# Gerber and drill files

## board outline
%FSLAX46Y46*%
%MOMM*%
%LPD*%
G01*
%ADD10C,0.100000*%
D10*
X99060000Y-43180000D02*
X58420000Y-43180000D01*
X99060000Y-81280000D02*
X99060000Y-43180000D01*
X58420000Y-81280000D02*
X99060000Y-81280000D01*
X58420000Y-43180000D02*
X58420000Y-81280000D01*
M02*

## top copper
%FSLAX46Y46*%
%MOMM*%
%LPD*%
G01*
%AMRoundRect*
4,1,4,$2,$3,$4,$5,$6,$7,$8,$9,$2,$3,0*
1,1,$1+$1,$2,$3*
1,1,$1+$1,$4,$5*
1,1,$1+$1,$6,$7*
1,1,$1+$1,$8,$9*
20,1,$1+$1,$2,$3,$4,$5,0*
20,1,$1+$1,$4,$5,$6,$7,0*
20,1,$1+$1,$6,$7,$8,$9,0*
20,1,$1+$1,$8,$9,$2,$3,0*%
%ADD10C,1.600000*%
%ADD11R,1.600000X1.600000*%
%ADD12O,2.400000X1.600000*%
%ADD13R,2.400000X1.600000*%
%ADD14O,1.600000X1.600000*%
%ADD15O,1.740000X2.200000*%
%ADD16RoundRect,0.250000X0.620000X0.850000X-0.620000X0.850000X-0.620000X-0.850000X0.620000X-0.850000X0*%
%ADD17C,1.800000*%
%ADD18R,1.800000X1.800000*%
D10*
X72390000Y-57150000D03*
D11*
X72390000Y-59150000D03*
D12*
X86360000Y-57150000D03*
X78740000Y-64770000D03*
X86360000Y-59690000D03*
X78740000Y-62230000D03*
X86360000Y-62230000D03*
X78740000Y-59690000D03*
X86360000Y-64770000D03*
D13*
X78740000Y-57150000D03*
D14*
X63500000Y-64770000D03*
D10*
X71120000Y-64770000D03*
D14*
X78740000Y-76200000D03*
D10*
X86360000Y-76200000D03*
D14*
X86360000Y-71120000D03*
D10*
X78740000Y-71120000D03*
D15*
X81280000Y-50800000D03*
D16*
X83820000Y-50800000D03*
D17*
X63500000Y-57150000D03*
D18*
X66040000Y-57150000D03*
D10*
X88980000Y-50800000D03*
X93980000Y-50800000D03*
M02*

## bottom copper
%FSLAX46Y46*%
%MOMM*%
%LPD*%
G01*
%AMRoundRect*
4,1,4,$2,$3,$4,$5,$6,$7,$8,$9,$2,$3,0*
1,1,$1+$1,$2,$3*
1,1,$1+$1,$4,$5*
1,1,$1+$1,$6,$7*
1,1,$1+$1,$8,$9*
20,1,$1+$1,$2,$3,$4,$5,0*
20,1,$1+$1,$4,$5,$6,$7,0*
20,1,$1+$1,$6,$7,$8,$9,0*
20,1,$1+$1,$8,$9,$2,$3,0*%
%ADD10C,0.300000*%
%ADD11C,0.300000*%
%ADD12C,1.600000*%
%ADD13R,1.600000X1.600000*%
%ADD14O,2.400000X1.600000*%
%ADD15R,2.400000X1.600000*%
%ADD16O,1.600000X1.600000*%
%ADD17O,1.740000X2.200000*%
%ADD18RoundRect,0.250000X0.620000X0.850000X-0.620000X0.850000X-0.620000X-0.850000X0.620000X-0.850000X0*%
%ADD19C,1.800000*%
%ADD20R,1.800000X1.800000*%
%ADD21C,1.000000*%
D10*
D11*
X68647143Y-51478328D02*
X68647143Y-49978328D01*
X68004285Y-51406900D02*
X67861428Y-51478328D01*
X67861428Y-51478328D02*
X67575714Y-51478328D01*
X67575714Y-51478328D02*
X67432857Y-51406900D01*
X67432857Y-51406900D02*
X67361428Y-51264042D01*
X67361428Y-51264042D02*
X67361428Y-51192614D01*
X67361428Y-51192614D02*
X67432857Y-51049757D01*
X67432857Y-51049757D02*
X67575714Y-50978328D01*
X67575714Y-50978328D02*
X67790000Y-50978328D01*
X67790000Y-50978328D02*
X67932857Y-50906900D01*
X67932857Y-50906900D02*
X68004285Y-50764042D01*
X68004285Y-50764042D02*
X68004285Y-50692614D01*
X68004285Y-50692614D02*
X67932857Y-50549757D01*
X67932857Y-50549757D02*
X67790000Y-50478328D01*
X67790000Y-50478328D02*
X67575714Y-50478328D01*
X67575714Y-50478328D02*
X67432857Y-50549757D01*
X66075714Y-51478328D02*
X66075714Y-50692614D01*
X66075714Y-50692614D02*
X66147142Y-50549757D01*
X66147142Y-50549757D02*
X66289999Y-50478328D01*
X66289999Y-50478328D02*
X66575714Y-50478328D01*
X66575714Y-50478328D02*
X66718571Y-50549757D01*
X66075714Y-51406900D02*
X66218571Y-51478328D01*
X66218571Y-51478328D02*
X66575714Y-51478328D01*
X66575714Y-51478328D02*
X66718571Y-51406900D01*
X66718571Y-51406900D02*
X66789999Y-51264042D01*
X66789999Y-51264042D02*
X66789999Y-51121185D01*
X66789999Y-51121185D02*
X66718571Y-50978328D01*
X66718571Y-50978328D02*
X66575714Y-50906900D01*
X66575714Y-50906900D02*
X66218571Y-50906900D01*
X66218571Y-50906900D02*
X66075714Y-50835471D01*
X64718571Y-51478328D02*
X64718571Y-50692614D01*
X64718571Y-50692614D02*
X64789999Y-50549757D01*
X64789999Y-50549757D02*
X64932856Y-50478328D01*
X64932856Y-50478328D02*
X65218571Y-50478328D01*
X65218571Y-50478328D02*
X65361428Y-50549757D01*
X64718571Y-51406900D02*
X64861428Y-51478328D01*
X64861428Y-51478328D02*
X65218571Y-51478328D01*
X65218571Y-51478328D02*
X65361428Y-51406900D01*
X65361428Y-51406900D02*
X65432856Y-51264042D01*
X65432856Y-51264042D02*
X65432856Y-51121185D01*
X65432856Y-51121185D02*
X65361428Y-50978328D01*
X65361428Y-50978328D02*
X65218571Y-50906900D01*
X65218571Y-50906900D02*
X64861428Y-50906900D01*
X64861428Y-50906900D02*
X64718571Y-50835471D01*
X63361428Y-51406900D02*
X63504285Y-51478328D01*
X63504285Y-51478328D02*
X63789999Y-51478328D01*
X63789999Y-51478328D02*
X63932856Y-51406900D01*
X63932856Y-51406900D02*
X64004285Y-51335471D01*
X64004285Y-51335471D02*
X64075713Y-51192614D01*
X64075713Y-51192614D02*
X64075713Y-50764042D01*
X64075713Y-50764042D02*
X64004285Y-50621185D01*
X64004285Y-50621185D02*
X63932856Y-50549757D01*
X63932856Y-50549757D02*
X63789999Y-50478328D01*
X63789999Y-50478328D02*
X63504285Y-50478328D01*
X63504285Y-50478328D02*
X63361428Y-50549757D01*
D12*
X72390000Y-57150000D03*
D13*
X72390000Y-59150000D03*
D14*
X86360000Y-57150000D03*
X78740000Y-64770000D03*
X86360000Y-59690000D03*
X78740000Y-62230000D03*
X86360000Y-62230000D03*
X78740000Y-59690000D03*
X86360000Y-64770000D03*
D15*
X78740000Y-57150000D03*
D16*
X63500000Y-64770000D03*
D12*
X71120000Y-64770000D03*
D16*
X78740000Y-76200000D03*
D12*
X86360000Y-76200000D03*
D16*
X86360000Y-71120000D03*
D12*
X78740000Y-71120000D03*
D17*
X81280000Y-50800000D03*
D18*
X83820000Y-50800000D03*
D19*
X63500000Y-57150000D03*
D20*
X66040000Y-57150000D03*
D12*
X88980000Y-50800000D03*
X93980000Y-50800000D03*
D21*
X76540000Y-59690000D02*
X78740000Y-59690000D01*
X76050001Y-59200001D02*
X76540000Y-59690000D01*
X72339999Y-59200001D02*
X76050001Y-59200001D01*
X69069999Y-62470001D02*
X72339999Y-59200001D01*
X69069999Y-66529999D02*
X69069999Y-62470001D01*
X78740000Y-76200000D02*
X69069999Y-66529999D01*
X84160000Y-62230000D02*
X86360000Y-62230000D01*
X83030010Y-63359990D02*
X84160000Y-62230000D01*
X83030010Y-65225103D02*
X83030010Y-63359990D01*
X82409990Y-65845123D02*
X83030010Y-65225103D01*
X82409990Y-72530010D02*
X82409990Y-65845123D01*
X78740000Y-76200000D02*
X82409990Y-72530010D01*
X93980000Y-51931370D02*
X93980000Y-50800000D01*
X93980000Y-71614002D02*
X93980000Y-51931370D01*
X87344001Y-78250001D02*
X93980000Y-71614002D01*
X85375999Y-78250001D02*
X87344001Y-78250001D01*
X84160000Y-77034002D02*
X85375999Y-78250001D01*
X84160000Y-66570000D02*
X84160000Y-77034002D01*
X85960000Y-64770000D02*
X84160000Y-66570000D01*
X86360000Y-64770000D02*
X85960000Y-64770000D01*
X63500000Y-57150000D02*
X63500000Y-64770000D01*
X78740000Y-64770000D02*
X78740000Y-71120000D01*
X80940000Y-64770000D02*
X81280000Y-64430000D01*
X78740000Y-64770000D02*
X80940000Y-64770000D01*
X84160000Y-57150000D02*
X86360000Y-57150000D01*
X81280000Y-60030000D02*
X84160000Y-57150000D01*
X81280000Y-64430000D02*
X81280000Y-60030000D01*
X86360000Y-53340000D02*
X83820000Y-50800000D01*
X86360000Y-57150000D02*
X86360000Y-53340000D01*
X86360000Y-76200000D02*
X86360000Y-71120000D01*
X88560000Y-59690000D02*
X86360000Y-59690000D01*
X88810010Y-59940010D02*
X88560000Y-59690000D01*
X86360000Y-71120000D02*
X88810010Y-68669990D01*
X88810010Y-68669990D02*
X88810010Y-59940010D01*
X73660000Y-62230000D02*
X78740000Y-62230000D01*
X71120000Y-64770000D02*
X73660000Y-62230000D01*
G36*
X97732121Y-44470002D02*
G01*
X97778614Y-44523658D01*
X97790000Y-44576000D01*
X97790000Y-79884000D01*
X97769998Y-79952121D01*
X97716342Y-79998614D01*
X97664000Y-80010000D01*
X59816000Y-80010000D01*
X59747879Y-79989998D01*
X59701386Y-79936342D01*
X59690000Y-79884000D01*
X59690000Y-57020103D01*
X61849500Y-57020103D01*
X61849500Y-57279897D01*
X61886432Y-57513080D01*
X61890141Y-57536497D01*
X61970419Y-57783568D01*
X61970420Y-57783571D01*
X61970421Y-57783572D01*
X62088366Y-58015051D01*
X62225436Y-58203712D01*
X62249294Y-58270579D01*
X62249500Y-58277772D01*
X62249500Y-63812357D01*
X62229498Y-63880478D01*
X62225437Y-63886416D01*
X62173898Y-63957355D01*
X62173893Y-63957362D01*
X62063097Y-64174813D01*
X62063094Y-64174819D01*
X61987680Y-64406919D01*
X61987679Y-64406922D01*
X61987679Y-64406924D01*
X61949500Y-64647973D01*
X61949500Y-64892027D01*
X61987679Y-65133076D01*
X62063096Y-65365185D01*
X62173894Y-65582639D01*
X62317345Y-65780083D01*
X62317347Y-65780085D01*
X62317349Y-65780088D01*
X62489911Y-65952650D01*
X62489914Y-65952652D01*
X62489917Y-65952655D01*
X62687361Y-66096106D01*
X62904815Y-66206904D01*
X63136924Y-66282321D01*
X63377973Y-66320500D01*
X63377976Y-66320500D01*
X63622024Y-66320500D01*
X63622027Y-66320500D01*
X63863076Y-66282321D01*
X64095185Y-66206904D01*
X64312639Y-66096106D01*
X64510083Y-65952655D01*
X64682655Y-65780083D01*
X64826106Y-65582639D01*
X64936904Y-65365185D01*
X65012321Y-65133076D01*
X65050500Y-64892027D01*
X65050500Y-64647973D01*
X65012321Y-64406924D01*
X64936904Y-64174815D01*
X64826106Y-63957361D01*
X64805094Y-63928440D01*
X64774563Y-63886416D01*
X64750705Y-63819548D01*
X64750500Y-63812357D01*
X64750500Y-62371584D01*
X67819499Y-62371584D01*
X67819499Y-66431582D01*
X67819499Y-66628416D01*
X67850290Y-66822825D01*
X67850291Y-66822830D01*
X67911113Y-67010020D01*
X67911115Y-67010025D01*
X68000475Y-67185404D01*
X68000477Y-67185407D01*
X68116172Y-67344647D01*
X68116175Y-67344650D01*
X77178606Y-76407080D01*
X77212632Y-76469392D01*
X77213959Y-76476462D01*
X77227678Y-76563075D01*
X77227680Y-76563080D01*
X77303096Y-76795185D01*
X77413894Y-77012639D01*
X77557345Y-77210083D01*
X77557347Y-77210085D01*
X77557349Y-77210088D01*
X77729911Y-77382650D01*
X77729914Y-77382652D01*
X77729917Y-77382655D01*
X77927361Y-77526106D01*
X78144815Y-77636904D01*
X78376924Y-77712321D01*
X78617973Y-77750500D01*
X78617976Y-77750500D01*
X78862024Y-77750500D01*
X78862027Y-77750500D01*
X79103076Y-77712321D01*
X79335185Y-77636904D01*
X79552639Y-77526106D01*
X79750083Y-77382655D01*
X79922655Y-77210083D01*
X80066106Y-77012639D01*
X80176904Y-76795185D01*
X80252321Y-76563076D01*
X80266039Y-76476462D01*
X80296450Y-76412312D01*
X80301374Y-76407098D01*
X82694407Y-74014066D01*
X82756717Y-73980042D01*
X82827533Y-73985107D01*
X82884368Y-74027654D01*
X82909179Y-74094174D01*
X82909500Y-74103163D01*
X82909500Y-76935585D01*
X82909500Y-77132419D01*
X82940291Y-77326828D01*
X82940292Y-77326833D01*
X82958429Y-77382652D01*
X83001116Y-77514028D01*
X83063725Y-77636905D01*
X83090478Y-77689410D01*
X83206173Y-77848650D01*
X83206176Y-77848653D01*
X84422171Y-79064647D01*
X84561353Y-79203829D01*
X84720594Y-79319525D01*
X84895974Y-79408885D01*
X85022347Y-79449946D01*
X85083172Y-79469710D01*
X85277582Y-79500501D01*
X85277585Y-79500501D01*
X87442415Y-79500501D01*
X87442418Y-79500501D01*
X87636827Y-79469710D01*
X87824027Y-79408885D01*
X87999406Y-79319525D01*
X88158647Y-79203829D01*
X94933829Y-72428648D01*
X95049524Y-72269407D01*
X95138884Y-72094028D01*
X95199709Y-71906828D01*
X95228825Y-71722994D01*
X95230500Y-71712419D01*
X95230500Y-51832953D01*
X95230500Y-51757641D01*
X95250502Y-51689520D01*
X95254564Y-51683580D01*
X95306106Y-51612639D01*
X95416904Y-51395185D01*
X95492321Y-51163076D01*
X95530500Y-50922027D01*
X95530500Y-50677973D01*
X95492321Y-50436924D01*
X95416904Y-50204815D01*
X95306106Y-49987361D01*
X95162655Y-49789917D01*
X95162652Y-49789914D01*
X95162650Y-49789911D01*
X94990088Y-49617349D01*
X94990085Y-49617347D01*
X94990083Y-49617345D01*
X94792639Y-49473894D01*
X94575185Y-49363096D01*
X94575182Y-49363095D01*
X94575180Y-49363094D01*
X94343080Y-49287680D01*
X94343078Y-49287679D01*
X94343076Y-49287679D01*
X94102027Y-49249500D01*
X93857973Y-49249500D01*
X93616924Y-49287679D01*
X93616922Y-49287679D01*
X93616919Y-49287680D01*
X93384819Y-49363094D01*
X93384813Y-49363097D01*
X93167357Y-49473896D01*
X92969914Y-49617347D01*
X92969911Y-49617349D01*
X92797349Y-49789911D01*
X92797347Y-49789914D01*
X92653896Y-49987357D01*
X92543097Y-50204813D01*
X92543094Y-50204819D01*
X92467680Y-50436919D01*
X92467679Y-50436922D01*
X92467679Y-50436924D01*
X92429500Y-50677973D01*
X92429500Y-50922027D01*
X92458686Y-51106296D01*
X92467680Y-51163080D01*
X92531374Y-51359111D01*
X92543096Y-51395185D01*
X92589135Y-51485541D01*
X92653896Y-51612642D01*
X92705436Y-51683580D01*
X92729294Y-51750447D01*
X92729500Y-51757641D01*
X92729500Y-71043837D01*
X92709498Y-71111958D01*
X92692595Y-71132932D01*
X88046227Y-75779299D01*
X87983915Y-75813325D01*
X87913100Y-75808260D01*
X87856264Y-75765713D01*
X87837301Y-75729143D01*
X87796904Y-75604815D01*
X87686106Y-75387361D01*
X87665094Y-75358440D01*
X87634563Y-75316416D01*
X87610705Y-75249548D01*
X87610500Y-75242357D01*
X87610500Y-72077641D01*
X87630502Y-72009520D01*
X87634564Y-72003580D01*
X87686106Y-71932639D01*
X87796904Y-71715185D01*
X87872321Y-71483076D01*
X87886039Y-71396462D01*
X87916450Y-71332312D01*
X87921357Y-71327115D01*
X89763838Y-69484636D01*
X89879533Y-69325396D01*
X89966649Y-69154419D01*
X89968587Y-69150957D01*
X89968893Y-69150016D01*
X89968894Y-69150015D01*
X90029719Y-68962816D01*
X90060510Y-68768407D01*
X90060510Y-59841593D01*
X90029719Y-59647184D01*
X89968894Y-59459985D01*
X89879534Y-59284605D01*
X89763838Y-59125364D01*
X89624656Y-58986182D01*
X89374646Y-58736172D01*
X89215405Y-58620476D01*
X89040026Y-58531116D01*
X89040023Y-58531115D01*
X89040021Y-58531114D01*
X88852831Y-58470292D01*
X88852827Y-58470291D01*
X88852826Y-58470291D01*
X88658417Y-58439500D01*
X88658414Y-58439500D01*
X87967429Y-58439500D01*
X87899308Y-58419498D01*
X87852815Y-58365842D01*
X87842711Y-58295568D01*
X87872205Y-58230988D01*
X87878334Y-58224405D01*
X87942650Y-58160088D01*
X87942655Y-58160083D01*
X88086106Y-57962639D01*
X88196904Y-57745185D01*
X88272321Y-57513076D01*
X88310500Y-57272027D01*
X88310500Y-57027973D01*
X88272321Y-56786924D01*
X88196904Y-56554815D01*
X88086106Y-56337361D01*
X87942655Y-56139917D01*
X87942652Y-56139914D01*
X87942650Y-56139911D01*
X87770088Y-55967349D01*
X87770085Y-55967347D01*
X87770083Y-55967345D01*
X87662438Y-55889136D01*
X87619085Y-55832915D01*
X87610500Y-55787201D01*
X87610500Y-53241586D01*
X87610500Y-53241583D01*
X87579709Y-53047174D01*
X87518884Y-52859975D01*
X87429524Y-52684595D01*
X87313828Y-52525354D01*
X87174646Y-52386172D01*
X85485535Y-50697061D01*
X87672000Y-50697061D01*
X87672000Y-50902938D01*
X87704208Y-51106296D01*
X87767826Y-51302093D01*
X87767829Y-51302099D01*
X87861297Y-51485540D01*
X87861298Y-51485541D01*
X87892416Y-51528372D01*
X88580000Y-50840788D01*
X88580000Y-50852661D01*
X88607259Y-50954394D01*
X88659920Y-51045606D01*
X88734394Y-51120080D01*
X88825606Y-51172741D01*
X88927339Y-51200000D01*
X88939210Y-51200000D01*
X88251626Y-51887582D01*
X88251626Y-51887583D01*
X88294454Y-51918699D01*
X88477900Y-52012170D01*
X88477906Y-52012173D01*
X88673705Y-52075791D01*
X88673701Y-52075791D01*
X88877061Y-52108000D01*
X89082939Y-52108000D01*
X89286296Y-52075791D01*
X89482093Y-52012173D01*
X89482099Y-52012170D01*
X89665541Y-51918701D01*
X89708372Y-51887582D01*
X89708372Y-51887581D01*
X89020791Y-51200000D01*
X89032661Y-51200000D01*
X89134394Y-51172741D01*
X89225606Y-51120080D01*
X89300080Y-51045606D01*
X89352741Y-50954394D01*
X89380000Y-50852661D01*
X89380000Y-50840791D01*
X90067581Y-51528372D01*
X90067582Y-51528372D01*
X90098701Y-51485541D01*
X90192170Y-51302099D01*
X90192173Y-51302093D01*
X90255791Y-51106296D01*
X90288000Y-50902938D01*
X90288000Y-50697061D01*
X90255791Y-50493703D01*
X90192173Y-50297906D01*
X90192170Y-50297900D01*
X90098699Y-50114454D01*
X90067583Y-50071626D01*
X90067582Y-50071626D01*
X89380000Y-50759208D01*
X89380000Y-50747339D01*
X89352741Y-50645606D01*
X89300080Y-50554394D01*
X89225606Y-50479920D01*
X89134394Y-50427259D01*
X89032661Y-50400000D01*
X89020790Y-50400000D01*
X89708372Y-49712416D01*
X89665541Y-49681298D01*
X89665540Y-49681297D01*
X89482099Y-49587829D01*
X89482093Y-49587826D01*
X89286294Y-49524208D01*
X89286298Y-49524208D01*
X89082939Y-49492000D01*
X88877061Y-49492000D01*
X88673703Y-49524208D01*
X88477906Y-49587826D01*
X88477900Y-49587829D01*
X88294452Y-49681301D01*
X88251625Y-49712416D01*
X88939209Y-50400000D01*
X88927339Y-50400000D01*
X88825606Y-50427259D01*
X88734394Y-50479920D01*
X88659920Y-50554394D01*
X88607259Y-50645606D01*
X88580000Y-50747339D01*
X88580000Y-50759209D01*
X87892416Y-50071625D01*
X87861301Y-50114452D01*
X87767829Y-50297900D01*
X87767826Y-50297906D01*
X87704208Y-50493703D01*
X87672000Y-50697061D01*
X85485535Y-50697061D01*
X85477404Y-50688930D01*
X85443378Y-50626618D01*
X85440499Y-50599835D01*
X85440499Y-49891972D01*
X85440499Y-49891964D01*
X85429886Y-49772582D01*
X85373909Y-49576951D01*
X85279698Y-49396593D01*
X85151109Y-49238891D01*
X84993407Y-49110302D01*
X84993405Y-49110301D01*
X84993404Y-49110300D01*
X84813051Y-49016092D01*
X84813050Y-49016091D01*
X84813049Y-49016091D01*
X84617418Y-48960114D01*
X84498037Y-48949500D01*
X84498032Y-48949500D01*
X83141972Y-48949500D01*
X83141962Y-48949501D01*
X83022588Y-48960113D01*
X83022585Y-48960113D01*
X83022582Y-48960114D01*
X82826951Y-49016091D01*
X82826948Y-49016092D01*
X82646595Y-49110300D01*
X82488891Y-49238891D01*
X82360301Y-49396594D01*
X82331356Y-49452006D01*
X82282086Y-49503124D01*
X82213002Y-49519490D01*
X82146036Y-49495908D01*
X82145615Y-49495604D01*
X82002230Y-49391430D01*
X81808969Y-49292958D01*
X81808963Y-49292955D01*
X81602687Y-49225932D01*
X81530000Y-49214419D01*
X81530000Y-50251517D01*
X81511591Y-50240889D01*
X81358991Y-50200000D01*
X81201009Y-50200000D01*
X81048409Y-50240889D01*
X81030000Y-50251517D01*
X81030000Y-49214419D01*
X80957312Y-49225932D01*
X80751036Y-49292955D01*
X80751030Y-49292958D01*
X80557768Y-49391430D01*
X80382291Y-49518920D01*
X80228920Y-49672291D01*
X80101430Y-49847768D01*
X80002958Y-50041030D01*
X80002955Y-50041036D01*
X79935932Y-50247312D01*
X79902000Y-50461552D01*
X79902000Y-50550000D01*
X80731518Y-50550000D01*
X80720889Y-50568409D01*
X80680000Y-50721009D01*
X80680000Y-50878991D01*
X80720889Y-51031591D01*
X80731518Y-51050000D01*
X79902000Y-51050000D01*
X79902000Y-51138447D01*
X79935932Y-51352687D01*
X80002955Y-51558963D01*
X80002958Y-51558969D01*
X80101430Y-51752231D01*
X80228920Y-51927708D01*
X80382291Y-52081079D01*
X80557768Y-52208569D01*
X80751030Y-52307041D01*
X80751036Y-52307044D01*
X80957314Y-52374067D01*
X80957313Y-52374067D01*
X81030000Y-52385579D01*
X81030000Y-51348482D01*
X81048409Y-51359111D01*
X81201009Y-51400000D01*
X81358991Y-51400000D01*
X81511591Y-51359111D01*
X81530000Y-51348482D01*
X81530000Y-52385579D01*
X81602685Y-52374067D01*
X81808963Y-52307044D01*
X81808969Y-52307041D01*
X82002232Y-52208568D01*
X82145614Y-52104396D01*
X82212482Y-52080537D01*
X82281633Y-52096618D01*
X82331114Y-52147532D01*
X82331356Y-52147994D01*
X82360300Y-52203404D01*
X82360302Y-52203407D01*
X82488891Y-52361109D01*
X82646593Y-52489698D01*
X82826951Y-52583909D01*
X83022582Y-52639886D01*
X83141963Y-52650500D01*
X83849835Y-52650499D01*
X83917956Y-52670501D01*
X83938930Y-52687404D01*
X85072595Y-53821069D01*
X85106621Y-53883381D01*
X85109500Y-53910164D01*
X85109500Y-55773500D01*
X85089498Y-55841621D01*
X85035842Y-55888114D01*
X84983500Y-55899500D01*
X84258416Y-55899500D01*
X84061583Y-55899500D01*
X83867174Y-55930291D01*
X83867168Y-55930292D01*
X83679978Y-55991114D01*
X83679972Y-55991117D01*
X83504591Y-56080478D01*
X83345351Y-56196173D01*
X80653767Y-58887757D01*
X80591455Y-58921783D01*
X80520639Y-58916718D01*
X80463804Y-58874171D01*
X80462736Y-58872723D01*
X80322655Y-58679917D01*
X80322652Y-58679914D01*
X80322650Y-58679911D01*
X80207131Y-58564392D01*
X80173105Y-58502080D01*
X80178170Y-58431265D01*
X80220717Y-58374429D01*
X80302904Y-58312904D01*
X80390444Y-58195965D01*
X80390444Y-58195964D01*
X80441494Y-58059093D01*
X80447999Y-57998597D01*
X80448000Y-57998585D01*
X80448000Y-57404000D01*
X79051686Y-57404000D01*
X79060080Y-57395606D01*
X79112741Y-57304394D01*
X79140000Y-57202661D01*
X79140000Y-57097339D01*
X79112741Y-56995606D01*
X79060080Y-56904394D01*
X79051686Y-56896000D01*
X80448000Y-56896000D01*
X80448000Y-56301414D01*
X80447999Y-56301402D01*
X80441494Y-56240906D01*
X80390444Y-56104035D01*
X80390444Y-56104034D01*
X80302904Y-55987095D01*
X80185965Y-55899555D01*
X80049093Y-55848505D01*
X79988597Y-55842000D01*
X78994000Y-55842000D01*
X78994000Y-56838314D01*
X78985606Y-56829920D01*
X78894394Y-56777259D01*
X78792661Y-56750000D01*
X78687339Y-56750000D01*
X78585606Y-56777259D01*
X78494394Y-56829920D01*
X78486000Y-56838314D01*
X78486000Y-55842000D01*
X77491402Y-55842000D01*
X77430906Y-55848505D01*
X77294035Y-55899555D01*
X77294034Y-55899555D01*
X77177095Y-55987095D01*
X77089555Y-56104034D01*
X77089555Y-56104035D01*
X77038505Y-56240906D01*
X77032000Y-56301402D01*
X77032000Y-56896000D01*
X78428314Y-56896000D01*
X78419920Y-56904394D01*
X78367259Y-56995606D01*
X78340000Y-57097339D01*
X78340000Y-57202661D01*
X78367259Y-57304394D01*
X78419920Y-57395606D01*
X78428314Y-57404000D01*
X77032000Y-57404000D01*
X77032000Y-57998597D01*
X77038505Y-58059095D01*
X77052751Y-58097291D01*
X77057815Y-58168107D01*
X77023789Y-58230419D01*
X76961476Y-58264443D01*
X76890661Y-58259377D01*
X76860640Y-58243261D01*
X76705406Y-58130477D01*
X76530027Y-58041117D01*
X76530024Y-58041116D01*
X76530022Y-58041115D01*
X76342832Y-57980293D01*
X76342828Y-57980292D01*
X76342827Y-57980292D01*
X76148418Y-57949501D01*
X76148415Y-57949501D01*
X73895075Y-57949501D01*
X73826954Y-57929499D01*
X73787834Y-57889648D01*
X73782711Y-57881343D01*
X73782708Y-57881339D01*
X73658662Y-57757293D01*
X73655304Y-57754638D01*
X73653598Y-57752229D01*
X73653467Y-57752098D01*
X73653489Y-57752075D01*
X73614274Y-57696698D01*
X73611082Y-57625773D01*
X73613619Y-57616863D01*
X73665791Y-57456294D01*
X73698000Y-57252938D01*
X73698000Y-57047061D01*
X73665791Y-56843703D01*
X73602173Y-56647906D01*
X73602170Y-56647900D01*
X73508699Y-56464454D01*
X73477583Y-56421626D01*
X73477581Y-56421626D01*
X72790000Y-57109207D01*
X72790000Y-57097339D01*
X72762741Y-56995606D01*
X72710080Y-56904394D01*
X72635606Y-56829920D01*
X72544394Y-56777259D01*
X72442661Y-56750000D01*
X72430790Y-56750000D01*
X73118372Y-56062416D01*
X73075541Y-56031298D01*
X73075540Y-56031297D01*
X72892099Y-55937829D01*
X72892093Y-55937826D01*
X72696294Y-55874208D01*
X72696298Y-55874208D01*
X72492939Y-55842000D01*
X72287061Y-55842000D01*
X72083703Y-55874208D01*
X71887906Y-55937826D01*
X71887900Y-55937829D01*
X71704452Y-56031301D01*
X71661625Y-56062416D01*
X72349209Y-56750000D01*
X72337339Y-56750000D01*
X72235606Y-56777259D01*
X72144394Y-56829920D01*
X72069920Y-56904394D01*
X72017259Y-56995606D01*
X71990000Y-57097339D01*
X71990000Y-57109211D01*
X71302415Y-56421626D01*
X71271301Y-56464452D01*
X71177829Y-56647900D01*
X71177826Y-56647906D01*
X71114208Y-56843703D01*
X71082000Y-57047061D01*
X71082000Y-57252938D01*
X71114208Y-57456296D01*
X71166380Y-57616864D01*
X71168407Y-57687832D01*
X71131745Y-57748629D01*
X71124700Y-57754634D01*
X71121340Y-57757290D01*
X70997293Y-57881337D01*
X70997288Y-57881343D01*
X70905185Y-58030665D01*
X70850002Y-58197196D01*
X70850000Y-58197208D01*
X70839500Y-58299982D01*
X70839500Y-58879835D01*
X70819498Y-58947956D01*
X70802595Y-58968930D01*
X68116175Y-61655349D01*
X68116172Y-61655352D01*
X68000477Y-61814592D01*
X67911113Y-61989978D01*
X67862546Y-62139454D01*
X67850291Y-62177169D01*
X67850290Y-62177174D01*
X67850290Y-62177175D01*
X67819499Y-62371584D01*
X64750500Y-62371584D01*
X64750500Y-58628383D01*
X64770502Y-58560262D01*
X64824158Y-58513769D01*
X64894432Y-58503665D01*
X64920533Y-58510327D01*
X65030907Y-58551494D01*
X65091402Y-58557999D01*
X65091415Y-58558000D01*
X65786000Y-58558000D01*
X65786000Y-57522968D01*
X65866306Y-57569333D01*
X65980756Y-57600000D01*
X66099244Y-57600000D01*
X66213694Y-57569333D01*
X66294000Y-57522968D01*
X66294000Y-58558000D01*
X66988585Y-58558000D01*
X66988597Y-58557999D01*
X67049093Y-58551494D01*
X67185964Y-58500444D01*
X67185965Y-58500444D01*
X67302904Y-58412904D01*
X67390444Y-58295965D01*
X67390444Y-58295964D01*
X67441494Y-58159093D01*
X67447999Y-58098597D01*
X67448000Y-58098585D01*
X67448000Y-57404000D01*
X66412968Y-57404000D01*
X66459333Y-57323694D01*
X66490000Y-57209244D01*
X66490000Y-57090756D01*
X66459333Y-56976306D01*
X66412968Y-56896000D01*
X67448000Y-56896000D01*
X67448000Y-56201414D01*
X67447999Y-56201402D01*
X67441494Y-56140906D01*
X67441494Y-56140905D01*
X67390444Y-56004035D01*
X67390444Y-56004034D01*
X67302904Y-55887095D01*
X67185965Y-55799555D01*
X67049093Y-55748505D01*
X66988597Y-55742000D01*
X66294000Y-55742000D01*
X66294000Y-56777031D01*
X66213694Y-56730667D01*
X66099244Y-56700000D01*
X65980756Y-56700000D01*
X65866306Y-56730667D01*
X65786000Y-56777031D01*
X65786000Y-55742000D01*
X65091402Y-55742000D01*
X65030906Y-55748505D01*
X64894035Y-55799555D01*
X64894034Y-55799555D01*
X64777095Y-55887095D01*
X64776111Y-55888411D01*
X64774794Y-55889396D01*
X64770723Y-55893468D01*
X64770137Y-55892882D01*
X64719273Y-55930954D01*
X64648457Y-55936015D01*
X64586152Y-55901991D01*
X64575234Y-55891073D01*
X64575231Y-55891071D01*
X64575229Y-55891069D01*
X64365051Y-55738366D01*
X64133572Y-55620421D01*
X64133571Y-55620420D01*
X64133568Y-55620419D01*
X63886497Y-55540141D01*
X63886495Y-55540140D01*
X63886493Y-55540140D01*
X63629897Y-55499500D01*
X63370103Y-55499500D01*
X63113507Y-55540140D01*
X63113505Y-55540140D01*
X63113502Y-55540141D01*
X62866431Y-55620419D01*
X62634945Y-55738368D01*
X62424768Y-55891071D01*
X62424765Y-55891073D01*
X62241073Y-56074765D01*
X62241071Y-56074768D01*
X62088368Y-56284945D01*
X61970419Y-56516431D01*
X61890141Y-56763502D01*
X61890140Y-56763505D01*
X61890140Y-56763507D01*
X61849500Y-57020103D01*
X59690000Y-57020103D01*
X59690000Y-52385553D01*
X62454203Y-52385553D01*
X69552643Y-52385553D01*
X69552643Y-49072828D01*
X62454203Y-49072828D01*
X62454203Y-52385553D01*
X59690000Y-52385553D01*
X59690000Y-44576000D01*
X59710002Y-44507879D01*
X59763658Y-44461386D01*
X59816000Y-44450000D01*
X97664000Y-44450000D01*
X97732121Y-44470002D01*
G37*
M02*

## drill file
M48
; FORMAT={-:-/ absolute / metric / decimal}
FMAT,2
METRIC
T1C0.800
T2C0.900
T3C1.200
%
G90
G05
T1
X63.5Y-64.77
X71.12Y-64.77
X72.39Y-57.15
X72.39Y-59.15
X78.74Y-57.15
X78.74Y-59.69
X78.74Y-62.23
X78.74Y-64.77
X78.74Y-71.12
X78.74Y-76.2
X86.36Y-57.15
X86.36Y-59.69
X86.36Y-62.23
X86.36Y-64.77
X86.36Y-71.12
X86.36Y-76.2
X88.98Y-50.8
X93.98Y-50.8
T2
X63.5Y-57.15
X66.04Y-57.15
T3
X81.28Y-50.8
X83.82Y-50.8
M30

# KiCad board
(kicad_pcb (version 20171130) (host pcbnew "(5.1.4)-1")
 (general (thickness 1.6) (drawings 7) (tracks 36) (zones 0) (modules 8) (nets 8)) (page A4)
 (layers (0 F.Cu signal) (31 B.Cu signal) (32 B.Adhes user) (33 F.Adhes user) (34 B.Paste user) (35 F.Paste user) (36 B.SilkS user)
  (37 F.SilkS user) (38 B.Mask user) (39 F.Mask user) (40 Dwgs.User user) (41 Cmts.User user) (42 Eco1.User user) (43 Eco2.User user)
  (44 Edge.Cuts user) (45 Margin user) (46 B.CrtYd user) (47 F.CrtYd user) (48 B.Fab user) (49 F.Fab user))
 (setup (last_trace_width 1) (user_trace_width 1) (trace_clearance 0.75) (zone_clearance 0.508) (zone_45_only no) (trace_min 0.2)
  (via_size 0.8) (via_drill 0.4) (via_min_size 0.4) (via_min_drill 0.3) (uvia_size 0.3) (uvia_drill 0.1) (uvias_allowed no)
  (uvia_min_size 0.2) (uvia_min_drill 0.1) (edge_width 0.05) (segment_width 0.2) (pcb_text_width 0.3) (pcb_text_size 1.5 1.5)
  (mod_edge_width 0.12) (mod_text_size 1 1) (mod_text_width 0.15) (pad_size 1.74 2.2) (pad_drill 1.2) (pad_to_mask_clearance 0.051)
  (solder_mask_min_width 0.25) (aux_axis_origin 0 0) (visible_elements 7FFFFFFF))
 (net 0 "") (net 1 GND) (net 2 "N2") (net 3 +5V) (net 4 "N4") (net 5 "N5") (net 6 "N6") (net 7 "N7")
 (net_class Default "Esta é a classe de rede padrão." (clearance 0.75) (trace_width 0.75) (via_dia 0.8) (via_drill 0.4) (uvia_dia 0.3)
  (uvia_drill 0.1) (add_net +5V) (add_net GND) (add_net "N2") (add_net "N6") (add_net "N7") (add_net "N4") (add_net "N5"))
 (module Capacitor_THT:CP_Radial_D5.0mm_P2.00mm (layer F.Cu) (at 72.39 59.15 90)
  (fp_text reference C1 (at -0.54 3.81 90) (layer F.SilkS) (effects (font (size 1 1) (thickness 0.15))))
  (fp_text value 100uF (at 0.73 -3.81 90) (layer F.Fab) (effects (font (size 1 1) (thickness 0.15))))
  (pad 2 thru_hole circle (at 2 0 90) (size 1.6 1.6) (drill 0.8) (layers *.Cu *.Mask) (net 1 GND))
  (pad 1 thru_hole rect (at 0 0 90) (size 1.6 1.6) (drill 0.8) (layers *.Cu *.Mask) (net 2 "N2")))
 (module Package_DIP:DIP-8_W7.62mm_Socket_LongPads (layer F.Cu) (at 78.74 57.15)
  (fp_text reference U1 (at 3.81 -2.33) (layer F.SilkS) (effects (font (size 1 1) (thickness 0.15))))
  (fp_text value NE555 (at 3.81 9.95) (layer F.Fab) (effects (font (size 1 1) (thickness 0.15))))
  (pad 8 thru_hole oval (at 7.62 0) (size 2.4 1.6) (drill 0.8) (layers *.Cu *.Mask) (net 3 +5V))
  (pad 4 thru_hole oval (at 0 7.62) (size 2.4 1.6) (drill 0.8) (layers *.Cu *.Mask) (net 3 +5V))
  (pad 7 thru_hole oval (at 7.62 2.54) (size 2.4 1.6) (drill 0.8) (layers *.Cu *.Mask) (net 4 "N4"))
  (pad 3 thru_hole oval (at 0 5.08) (size 2.4 1.6) (drill 0.8) (layers *.Cu *.Mask) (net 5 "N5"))
  (pad 6 thru_hole oval (at 7.62 5.08) (size 2.4 1.6) (drill 0.8) (layers *.Cu *.Mask) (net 2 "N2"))
  (pad 2 thru_hole oval (at 0 2.54) (size 2.4 1.6) (drill 0.8) (layers *.Cu *.Mask) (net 2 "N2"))
  (pad 5 thru_hole oval (at 7.62 7.62) (size 2.4 1.6) (drill 0.8) (layers *.Cu *.Mask) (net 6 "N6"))
  (pad 1 thru_hole rect (at 0 0) (size 2.4 1.6) (drill 0.8) (layers *.Cu *.Mask) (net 1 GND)))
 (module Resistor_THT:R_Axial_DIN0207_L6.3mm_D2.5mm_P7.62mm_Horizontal (layer F.Cu) (at 71.12 64.77 180)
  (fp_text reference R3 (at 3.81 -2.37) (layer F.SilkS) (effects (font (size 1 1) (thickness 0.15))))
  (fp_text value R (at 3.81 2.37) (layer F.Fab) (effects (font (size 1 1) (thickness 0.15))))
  (pad 2 thru_hole oval (at 7.62 0 180) (size 1.6 1.6) (drill 0.8) (layers *.Cu *.Mask) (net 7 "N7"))
  (pad 1 thru_hole circle (at 0 0 180) (size 1.6 1.6) (drill 0.8) (layers *.Cu *.Mask) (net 5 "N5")))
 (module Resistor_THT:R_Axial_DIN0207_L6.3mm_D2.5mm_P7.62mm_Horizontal (layer F.Cu) (at 86.36 76.2 180)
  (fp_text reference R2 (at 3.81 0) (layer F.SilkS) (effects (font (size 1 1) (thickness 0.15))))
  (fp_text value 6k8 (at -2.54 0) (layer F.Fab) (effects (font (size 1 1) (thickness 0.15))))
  (pad 2 thru_hole oval (at 7.62 0 180) (size 1.6 1.6) (drill 0.8) (layers *.Cu *.Mask) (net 2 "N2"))
  (pad 1 thru_hole circle (at 0 0 180) (size 1.6 1.6) (drill 0.8) (layers *.Cu *.Mask) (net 4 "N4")))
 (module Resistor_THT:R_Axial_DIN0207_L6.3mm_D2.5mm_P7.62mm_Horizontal (layer F.Cu) (at 78.74 71.12)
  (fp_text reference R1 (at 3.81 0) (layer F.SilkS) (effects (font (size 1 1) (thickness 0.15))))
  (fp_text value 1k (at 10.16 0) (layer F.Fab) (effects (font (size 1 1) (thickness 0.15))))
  (pad 2 thru_hole oval (at 7.62 0) (size 1.6 1.6) (drill 0.8) (layers *.Cu *.Mask) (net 4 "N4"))
  (pad 1 thru_hole circle (at 0 0) (size 1.6 1.6) (drill 0.8) (layers *.Cu *.Mask) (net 3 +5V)))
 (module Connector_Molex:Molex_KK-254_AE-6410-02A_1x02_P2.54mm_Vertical (layer F.Cu) (at 83.82 50.8 180)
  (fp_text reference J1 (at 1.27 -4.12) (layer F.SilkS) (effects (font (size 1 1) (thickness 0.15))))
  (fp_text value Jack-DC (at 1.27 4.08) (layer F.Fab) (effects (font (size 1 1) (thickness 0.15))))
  (pad 2 thru_hole oval (at 2.54 0 180) (size 1.74 2.2) (drill 1.2) (layers *.Cu *.Mask) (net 1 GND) (thermal_width 0.5))
  (pad 1 thru_hole roundrect (at 0 0 180) (size 1.74 2.2) (drill 1.2) (layers *.Cu *.Mask) (roundrect_rratio 0.143678) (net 3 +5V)))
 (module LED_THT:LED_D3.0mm (layer F.Cu) (at 66.04 57.15 180)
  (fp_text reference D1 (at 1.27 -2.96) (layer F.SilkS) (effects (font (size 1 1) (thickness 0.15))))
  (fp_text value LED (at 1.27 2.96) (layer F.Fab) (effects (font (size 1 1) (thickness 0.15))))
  (pad 2 thru_hole circle (at 2.54 0 180) (size 1.8 1.8) (drill 0.9) (layers *.Cu *.Mask) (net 7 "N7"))
  (pad 1 thru_hole rect (at 0 0 180) (size 1.8 1.8) (drill 0.9) (layers *.Cu *.Mask) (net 1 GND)))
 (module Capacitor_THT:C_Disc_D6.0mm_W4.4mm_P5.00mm (layer F.Cu) (at 93.98 50.8 180)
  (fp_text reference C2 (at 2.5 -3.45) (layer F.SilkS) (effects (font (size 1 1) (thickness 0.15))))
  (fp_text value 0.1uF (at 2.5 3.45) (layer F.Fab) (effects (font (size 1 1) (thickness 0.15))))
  (pad 2 thru_hole circle (at 5 0 180) (size 1.6 1.6) (drill 0.8) (layers *.Cu *.Mask) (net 1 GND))
  (pad 1 thru_hole circle (at 0 0 180) (size 1.6 1.6) (drill 0.8) (layers *.Cu *.Mask) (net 6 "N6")))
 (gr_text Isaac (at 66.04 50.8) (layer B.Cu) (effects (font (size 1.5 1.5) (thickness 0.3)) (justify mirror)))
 (gr_line (start 99.06 43.18) (end 58.42 43.18) (layer Edge.Cuts) (width 0.1))
 (gr_line (start 99.06 81.28) (end 99.06 43.18) (layer Edge.Cuts) (width 0.1))
 (gr_line (start 58.42 81.28) (end 99.06 81.28) (layer Edge.Cuts) (width 0.1))
 (gr_line (start 58.42 43.18) (end 58.42 81.28) (layer Edge.Cuts) (width 0.1))
 (segment (start 76.54 59.69) (end 78.74 59.69) (width 1) (layer B.Cu) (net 2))
 (segment (start 76.050001 59.200001) (end 76.54 59.69) (width 1) (layer B.Cu) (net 2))
 (segment (start 72.339999 59.200001) (end 76.050001 59.200001) (width 1) (layer B.Cu) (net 2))
 (segment (start 69.069999 62.470001) (end 72.339999 59.200001) (width 1) (layer B.Cu) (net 2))
 (segment (start 69.069999 66.529999) (end 69.069999 62.470001) (width 1) (layer B.Cu) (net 2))
 (segment (start 78.74 76.2) (end 69.069999 66.529999) (width 1) (layer B.Cu) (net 2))
 (segment (start 84.16 62.23) (end 86.36 62.23) (width 1) (layer B.Cu) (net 2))
 (segment (start 83.03001 63.35999) (end 84.16 62.23) (width 1) (layer B.Cu) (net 2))
 (segment (start 83.03001 65.225103) (end 83.03001 63.35999) (width 1) (layer B.Cu) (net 2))
 (segment (start 82.40999 65.845123) (end 83.03001 65.225103) (width 1) (layer B.Cu) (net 2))
 (segment (start 82.40999 72.53001) (end 82.40999 65.845123) (width 1) (layer B.Cu) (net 2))
 (segment (start 78.74 76.2) (end 82.40999 72.53001) (width 1) (layer B.Cu) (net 2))
 (segment (start 93.98 51.93137) (end 93.98 50.8) (width 1) (layer B.Cu) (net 6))
 (segment (start 93.98 71.614002) (end 93.98 51.93137) (width 1) (layer B.Cu) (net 6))
 (segment (start 87.344001 78.250001) (end 93.98 71.614002) (width 1) (layer B.Cu) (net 6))
 (segment (start 85.375999 78.250001) (end 87.344001 78.250001) (width 1) (layer B.Cu) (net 6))
 (segment (start 84.16 77.034002) (end 85.375999 78.250001) (width 1) (layer B.Cu) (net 6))
 (segment (start 84.16 66.57) (end 84.16 77.034002) (width 1) (layer B.Cu) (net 6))
 (segment (start 85.96 64.77) (end 84.16 66.57) (width 1) (layer B.Cu) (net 6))
 (segment (start 86.36 64.77) (end 85.96 64.77) (width 1) (layer B.Cu) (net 6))
 (segment (start 63.5 57.15) (end 63.5 64.77) (width 1) (layer B.Cu) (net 7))
 (segment (start 78.74 64.77) (end 78.74 71.12) (width 1) (layer B.Cu) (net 3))
 (segment (start 80.94 64.77) (end 81.28 64.43) (width 1) (layer B.Cu) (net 3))
 (segment (start 78.74 64.77) (end 80.94 64.77) (width 1) (layer B.Cu) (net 3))
 (segment (start 84.16 57.15) (end 86.36 57.15) (width 1) (layer B.Cu) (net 3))
 (segment (start 81.28 60.03) (end 84.16 57.15) (width 1) (layer B.Cu) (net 3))
 (segment (start 81.28 64.43) (end 81.28 60.03) (width 1) (layer B.Cu) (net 3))
 (segment (start 86.36 53.34) (end 83.82 50.8) (width 1) (layer B.Cu) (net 3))
 (segment (start 86.36 57.15) (end 86.36 53.34) (width 1) (layer B.Cu) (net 3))
 (segment (start 86.36 76.2) (end 86.36 71.12) (width 1) (layer B.Cu) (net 4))
 (segment (start 88.56 59.69) (end 86.36 59.69) (width 1) (layer B.Cu) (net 4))
 (segment (start 88.81001 59.94001) (end 88.56 59.69) (width 1) (layer B.Cu) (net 4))
 (segment (start 86.36 71.12) (end 88.81001 68.66999) (width 1) (layer B.Cu) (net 4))
 (segment (start 88.81001 68.66999) (end 88.81001 59.94001) (width 1) (layer B.Cu) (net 4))
 (segment (start 73.66 62.23) (end 78.74 62.23) (width 1) (layer B.Cu) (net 5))
 (segment (start 71.12 64.77) (end 73.66 62.23) (width 1) (layer B.Cu) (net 5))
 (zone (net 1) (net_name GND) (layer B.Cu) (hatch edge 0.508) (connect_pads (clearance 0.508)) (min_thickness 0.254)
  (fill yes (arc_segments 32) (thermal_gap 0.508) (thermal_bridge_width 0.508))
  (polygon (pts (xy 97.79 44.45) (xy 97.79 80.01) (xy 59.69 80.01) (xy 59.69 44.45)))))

